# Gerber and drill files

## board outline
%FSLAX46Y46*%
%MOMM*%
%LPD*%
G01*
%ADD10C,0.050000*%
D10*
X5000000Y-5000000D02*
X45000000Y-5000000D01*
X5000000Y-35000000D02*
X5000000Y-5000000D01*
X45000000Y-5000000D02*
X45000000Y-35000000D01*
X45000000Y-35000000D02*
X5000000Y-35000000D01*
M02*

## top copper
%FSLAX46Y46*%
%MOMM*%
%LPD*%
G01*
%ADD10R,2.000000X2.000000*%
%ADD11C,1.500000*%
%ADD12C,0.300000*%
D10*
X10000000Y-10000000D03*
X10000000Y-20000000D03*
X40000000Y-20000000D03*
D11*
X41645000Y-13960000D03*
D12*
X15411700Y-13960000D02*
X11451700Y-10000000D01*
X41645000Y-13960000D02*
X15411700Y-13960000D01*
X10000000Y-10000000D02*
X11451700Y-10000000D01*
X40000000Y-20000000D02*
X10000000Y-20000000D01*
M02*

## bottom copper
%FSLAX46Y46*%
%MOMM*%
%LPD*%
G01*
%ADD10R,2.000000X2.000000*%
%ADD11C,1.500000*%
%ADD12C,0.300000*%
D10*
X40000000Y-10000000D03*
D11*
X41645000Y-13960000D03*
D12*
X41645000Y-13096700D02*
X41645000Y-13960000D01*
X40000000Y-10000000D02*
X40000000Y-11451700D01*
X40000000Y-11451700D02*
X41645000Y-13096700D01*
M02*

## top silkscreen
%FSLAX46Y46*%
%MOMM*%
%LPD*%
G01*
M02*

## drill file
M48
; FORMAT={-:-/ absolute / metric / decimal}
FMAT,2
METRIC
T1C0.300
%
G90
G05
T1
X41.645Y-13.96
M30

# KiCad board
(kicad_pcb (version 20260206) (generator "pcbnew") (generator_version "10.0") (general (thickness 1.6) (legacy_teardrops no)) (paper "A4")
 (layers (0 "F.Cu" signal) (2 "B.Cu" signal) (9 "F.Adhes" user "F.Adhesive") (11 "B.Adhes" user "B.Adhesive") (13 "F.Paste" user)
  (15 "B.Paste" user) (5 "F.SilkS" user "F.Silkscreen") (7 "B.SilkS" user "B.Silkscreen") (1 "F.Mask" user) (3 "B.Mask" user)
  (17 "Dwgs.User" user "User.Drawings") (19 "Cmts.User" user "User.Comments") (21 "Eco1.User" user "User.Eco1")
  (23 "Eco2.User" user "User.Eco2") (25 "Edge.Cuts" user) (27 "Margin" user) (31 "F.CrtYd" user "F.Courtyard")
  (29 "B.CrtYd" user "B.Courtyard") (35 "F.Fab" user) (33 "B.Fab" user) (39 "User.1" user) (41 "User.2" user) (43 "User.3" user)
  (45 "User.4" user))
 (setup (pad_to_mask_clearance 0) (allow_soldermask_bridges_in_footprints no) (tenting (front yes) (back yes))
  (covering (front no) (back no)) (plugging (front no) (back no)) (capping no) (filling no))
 (gr_line (start 5 5) (end 45 5) (stroke (width 0.05) (type default)) (layer "Edge.Cuts"))
 (gr_line (start 5 35) (end 5 5) (stroke (width 0.05) (type default)) (layer "Edge.Cuts"))
 (gr_line (start 45 5) (end 45 35) (stroke (width 0.05) (type default)) (layer "Edge.Cuts"))
 (gr_line (start 45 35) (end 5 35) (stroke (width 0.05) (type default)) (layer "Edge.Cuts"))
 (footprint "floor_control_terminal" (layer "F.Cu") (at 10 10)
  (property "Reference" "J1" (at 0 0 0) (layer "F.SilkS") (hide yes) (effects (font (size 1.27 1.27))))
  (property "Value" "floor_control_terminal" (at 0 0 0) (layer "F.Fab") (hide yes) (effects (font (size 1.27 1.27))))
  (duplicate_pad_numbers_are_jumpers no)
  (pad "1" smd rect (at 0 0) (size 2 2) (layers "F.Cu" "F.Paste" "F.Mask") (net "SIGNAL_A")))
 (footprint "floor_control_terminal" (layer "B.Cu") (at 40 10)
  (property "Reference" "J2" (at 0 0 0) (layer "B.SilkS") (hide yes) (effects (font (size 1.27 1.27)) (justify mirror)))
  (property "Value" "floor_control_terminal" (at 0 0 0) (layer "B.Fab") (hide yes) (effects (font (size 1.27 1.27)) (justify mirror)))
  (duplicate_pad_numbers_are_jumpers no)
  (pad "1" smd rect (at 0 0) (size 2 2) (layers "B.Cu" "B.Paste" "B.Mask") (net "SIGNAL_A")))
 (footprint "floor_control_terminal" (layer "F.Cu") (at 10 20)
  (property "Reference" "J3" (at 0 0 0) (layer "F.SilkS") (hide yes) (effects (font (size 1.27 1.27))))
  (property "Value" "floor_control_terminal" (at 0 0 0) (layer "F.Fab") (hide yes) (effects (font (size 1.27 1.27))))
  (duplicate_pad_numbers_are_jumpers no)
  (pad "1" smd rect (at 0 0) (size 2 2) (layers "F.Cu" "F.Paste" "F.Mask") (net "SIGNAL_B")))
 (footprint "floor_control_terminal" (layer "F.Cu") (at 40 20)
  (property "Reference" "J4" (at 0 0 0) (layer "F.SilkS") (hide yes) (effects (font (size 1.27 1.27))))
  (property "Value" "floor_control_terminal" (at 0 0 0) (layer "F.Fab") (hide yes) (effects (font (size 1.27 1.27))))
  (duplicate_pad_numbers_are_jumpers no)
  (pad "1" smd rect (at 0 0) (size 2 2) (layers "F.Cu" "F.Paste" "F.Mask") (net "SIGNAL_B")))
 (segment (start 15.4117 13.96) (end 11.4517 10) (width 0.3) (layer "F.Cu") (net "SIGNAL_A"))
 (segment (start 41.645 13.96) (end 15.4117 13.96) (width 0.3) (layer "F.Cu") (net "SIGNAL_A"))
 (segment (start 10 10) (end 11.4517 10) (width 0.3) (layer "F.Cu") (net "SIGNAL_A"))
 (via (at 41.645 13.96) (size 1.5) (drill 0.3) (layers "F.Cu" "B.Cu") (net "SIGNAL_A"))
 (segment (start 41.645 13.0967) (end 41.645 13.96) (width 0.3) (layer "B.Cu") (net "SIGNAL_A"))
 (segment (start 40 10) (end 40 11.4517) (width 0.3) (layer "B.Cu") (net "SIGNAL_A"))
 (segment (start 40 11.4517) (end 41.645 13.0967) (width 0.3) (layer "B.Cu") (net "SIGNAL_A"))
 (segment (start 40 20) (end 10 20) (width 0.3) (layer "F.Cu") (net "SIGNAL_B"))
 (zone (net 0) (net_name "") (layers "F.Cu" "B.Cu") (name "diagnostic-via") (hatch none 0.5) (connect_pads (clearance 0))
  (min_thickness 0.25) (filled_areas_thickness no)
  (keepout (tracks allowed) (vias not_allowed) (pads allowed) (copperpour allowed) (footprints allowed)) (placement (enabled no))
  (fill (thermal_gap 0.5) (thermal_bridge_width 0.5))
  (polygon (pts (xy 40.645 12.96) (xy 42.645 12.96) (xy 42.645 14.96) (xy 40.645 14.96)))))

